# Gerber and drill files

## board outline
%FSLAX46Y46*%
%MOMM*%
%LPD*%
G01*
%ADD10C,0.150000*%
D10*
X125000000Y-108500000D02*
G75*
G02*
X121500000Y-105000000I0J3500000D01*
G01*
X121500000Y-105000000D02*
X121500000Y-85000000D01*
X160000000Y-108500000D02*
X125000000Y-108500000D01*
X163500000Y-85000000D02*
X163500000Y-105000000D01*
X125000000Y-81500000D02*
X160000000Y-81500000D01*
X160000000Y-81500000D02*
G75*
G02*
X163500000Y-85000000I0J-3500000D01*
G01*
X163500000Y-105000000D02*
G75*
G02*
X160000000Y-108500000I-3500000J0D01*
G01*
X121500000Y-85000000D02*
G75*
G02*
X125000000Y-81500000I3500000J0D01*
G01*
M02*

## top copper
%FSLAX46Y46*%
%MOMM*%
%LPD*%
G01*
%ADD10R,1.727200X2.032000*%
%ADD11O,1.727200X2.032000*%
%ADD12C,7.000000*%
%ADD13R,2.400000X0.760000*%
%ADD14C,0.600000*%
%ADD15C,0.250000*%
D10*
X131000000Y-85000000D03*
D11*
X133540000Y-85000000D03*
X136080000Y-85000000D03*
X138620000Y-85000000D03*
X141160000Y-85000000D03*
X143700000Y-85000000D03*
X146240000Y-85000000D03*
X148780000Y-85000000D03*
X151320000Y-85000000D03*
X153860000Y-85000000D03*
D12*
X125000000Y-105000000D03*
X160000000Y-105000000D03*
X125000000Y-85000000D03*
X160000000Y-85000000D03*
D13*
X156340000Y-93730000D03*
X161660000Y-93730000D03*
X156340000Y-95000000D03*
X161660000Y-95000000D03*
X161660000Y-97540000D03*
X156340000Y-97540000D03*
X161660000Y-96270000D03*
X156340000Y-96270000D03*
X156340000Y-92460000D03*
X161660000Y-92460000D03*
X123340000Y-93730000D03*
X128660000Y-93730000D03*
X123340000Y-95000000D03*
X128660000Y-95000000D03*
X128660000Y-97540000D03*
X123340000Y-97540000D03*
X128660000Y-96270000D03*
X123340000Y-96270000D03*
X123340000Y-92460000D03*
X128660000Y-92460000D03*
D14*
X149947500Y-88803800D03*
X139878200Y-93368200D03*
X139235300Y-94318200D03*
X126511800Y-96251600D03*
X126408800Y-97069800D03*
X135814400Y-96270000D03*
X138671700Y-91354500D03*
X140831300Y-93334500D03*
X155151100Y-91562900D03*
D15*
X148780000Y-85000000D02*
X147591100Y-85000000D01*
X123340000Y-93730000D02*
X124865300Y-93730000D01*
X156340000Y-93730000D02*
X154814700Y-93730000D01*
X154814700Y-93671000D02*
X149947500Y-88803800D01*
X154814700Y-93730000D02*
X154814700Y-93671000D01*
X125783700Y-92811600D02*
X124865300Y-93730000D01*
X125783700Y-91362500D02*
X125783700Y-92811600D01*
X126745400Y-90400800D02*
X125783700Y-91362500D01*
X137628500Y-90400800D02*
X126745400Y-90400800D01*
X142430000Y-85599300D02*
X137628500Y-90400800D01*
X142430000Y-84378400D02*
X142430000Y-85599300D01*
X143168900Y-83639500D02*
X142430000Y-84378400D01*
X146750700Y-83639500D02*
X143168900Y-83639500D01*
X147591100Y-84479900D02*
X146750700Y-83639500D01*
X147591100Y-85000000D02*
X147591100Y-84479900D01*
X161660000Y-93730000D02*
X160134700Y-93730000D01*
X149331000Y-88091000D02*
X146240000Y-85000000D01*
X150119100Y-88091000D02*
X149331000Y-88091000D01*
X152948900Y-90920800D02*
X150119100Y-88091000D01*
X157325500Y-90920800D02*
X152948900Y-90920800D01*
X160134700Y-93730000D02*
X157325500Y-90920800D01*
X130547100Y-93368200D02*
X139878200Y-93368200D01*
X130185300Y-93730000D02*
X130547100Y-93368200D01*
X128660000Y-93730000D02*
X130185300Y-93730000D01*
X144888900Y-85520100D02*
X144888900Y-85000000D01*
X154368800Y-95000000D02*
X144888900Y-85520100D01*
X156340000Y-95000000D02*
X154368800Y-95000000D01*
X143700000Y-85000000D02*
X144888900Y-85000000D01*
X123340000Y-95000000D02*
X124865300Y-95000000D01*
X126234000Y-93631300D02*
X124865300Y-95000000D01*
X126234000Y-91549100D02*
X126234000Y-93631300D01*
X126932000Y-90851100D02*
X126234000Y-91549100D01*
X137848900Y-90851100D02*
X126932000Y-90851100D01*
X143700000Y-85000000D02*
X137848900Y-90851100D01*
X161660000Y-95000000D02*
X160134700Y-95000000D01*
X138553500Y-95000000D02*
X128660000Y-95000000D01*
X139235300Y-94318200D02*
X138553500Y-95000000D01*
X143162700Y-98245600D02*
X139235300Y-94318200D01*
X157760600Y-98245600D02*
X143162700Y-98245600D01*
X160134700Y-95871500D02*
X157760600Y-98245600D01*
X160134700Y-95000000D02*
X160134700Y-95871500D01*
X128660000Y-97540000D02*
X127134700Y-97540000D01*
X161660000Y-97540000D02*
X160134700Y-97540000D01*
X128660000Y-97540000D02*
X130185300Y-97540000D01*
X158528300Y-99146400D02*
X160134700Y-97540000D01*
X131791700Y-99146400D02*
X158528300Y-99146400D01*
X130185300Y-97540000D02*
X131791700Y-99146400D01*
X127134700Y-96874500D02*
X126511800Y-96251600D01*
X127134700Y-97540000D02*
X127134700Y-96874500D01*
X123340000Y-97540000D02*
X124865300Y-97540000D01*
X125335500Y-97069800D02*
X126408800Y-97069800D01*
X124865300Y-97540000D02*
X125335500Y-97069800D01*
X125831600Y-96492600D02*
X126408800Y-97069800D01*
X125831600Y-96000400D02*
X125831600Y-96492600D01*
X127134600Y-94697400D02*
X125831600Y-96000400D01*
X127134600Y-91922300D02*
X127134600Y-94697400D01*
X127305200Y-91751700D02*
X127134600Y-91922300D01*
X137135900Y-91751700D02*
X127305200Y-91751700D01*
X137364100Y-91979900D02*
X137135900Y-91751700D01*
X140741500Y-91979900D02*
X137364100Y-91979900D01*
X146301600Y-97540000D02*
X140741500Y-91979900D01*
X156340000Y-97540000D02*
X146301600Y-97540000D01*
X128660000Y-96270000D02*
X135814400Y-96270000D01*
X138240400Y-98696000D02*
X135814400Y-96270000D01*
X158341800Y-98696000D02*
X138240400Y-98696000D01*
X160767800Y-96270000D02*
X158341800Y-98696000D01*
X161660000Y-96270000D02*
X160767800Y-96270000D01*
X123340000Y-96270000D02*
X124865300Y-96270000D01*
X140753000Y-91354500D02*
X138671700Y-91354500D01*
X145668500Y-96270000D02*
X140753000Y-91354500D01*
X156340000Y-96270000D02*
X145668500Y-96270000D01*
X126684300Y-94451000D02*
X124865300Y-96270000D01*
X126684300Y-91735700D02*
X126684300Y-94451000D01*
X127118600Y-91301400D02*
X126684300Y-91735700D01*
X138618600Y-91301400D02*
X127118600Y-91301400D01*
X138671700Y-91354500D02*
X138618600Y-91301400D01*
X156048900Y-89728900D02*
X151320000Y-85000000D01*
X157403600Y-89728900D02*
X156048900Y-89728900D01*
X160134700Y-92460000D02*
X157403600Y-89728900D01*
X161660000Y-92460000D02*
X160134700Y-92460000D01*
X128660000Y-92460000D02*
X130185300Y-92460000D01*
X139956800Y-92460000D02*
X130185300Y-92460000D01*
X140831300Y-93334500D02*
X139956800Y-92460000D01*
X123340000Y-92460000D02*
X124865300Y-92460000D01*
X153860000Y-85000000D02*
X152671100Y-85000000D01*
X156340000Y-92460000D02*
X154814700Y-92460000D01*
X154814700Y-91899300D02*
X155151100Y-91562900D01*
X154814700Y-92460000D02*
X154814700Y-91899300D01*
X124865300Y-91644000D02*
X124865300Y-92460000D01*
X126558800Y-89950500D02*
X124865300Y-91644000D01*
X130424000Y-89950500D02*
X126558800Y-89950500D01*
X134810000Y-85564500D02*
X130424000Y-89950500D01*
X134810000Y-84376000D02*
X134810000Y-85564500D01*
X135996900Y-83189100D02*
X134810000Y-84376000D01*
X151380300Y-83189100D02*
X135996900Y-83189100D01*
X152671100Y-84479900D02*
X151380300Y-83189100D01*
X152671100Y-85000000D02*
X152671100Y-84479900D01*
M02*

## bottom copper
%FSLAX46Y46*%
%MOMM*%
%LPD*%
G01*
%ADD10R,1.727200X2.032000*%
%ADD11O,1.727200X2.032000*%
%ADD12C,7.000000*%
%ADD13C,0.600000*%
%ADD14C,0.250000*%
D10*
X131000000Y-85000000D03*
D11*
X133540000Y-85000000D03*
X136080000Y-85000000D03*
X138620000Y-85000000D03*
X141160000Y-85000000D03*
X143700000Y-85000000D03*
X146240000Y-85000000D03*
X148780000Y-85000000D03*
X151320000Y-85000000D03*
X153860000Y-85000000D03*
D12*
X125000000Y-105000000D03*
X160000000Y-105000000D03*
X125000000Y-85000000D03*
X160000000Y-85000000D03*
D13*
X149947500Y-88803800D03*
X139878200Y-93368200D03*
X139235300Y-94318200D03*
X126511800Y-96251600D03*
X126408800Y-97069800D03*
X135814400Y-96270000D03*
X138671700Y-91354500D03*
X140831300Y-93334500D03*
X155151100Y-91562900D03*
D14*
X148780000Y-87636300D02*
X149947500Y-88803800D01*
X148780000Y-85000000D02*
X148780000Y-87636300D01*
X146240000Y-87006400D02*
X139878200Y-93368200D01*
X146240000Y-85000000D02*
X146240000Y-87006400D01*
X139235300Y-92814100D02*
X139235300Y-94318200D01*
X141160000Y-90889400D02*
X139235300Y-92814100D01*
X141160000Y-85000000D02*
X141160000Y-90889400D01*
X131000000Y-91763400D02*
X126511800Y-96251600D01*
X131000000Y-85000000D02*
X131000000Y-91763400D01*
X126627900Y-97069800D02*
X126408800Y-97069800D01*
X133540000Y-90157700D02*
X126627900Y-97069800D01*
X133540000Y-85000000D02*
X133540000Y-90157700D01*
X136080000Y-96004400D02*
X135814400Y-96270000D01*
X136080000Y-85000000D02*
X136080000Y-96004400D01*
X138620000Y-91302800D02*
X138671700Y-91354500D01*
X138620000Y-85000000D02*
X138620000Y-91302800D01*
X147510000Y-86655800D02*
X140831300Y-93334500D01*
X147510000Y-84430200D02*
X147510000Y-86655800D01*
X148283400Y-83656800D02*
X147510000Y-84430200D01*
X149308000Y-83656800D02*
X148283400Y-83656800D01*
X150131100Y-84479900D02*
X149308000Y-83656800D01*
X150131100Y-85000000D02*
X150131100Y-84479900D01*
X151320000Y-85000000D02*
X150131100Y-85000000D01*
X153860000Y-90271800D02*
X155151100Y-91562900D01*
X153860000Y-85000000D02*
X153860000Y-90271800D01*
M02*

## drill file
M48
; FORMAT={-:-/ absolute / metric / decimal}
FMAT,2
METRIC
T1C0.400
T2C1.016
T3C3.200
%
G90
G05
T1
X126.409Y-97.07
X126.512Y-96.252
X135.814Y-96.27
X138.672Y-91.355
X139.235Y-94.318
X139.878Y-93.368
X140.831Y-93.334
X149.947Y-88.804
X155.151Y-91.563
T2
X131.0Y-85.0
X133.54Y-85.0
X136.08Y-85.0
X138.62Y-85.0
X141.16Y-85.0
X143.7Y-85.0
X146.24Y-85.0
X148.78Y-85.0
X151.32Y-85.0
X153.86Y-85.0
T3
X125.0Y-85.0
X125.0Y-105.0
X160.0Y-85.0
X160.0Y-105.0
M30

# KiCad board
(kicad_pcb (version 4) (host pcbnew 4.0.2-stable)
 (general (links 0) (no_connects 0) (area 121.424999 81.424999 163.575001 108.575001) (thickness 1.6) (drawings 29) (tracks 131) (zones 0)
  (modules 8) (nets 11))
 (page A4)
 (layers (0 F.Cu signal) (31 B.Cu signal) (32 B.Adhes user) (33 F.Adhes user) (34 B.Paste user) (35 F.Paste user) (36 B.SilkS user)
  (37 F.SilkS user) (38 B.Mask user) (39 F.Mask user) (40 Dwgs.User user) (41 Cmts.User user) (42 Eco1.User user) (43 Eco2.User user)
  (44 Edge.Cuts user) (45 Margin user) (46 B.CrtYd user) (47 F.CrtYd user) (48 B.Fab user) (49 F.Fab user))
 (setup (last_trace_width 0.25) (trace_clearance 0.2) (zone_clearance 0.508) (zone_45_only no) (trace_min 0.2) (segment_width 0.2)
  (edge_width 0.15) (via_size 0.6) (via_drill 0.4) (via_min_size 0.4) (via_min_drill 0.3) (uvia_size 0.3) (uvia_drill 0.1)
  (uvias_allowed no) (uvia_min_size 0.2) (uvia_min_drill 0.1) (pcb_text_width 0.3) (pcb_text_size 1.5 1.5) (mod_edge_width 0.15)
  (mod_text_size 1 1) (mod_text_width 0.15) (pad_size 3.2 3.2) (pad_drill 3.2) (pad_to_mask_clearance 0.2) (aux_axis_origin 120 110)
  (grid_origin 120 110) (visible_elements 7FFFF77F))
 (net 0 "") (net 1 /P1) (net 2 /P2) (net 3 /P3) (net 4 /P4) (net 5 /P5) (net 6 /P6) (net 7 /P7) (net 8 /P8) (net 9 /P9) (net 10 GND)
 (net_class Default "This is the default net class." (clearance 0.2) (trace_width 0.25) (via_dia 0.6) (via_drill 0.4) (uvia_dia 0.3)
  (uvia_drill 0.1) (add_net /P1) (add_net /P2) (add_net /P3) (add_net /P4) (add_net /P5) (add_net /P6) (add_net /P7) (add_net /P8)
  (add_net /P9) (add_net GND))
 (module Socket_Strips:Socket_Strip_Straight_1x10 (layer F.Cu) (at 131 85)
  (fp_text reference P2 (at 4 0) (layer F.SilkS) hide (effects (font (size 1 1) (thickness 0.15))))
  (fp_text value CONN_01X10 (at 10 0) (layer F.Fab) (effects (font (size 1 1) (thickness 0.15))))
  (pad 1 thru_hole rect (at 0 0) (size 1.7272 2.032) (drill 1.016) (layers *.Cu *.Mask F.SilkS) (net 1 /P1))
  (pad 2 thru_hole oval (at 2.54 0) (size 1.7272 2.032) (drill 1.016) (layers *.Cu *.Mask F.SilkS) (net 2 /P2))
  (pad 3 thru_hole oval (at 5.08 0) (size 1.7272 2.032) (drill 1.016) (layers *.Cu *.Mask F.SilkS) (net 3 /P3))
  (pad 4 thru_hole oval (at 7.62 0) (size 1.7272 2.032) (drill 1.016) (layers *.Cu *.Mask F.SilkS) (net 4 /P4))
  (pad 5 thru_hole oval (at 10.16 0) (size 1.7272 2.032) (drill 1.016) (layers *.Cu *.Mask F.SilkS) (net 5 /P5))
  (pad 6 thru_hole oval (at 12.7 0) (size 1.7272 2.032) (drill 1.016) (layers *.Cu *.Mask F.SilkS) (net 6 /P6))
  (pad 7 thru_hole oval (at 15.24 0) (size 1.7272 2.032) (drill 1.016) (layers *.Cu *.Mask F.SilkS) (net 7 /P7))
  (pad 8 thru_hole oval (at 17.78 0) (size 1.7272 2.032) (drill 1.016) (layers *.Cu *.Mask F.SilkS) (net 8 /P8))
  (pad 9 thru_hole oval (at 20.32 0) (size 1.7272 2.032) (drill 1.016) (layers *.Cu *.Mask F.SilkS) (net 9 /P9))
  (pad 10 thru_hole oval (at 22.86 0) (size 1.7272 2.032) (drill 1.016) (layers *.Cu *.Mask F.SilkS) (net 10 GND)))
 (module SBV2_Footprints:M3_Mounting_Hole (layer F.Cu) (at 125 105)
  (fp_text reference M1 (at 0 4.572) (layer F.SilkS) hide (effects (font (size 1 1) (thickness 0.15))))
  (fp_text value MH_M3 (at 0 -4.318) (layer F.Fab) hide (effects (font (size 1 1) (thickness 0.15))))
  (pad "" np_thru_hole circle (at 0 0) (size 7 7) (drill 3.2) (layers *.Cu *.Mask)))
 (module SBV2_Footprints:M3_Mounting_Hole (layer F.Cu) (at 160 105)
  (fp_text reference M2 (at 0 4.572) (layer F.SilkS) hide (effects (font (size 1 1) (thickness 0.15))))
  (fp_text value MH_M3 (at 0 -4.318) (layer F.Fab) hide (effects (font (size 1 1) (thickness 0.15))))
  (pad "" np_thru_hole circle (at 0 0) (size 7 7) (drill 3.2) (layers *.Cu *.Mask)))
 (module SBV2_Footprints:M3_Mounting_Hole (layer F.Cu) (at 125 85)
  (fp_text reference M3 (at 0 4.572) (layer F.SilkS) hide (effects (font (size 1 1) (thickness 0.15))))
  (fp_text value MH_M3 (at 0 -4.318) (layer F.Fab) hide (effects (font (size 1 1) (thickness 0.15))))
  (pad "" np_thru_hole circle (at 0 0) (size 7 7) (drill 3.2) (layers *.Cu *.Mask)))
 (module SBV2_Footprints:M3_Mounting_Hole (layer F.Cu) (at 160 85)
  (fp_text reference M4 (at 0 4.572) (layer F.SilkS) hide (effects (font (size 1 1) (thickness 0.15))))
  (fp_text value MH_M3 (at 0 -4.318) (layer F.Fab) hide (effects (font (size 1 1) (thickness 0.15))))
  (pad "" np_thru_hole circle (at 0 0) (size 7 7) (drill 3.2) (layers *.Cu *.Mask)))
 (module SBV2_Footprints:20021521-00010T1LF (layer F.Cu) (at 159 95 90)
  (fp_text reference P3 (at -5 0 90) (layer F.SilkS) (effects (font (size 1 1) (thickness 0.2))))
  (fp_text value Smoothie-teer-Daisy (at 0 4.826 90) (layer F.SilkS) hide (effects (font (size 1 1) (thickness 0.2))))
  (pad 8 smd rect (at 1.27 -2.66 90) (size 0.76 2.4) (layers F.Cu F.Paste F.Mask) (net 8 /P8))
  (pad 7 smd rect (at 1.27 2.66 90) (size 0.76 2.4) (layers F.Cu F.Paste F.Mask) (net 7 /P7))
  (pad 6 smd rect (at 0 -2.66 90) (size 0.76 2.4) (layers F.Cu F.Paste F.Mask) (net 6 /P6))
  (pad 5 smd rect (at 0 2.66 270) (size 0.76 2.4) (layers F.Cu F.Paste F.Mask) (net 5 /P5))
  (pad 1 smd rect (at -2.54 2.66 90) (size 0.76 2.4) (layers F.Cu F.Paste F.Mask) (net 1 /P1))
  (pad 2 smd rect (at -2.54 -2.66 90) (size 0.76 2.4) (layers F.Cu F.Paste F.Mask) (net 2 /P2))
  (pad 3 smd rect (at -1.27 2.66 90) (size 0.76 2.4) (layers F.Cu F.Paste F.Mask) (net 3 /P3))
  (pad 4 smd rect (at -1.27 -2.66 90) (size 0.76 2.4) (layers F.Cu F.Paste F.Mask) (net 4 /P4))
  (pad 10 smd rect (at 2.54 -2.66 90) (size 0.76 2.4) (layers F.Cu F.Paste F.Mask) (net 10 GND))
  (pad 9 smd rect (at 2.54 2.66 90) (size 0.76 2.4) (layers F.Cu F.Paste F.Mask) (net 9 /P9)))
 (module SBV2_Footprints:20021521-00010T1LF (layer F.Cu) (at 126 95 90)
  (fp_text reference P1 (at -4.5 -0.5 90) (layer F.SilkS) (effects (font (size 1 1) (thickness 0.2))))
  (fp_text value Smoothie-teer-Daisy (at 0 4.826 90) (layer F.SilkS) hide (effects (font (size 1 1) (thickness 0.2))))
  (pad 8 smd rect (at 1.27 -2.66 90) (size 0.76 2.4) (layers F.Cu F.Paste F.Mask) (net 8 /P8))
  (pad 7 smd rect (at 1.27 2.66 90) (size 0.76 2.4) (layers F.Cu F.Paste F.Mask) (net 7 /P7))
  (pad 6 smd rect (at 0 -2.66 90) (size 0.76 2.4) (layers F.Cu F.Paste F.Mask) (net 6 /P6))
  (pad 5 smd rect (at 0 2.66 270) (size 0.76 2.4) (layers F.Cu F.Paste F.Mask) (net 5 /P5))
  (pad 1 smd rect (at -2.54 2.66 90) (size 0.76 2.4) (layers F.Cu F.Paste F.Mask) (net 1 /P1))
  (pad 2 smd rect (at -2.54 -2.66 90) (size 0.76 2.4) (layers F.Cu F.Paste F.Mask) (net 2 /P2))
  (pad 3 smd rect (at -1.27 2.66 90) (size 0.76 2.4) (layers F.Cu F.Paste F.Mask) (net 3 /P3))
  (pad 4 smd rect (at -1.27 -2.66 90) (size 0.76 2.4) (layers F.Cu F.Paste F.Mask) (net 4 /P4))
  (pad 10 smd rect (at 2.54 -2.66 90) (size 0.76 2.4) (layers F.Cu F.Paste F.Mask) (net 10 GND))
  (pad 9 smd rect (at 2.54 2.66 90) (size 0.76 2.4) (layers F.Cu F.Paste F.Mask) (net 9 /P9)))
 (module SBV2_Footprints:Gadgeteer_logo (layer F.Cu) (at 143 98.25)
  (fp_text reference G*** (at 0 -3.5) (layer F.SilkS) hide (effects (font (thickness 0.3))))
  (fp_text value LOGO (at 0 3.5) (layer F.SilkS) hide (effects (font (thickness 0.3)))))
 (gr_arc (start 125 105) (end 125 108.5) (angle 90) (layer Edge.Cuts) (width 0.15))
 (gr_line (start 121.5 105) (end 121.5 85) (angle 90) (layer Edge.Cuts) (width 0.15))
 (gr_line (start 160 108.5) (end 125 108.5) (angle 90) (layer Edge.Cuts) (width 0.15))
 (gr_line (start 163.5 85) (end 163.5 105) (angle 90) (layer Edge.Cuts) (width 0.15))
 (gr_line (start 125 81.5) (end 160 81.5) (angle 90) (layer Edge.Cuts) (width 0.15))
 (gr_arc (start 160 85) (end 160 81.5) (angle 90) (layer Edge.Cuts) (width 0.15))
 (gr_arc (start 160 105) (end 163.5 105) (angle 90) (layer Edge.Cuts) (width 0.15))
 (gr_arc (start 125 85) (end 121.5 85) (angle 90) (layer Edge.Cuts) (width 0.15))
 (via (at 149.9475 88.8038) (size 0.6) (layers F.Cu B.Cu) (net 8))
 (segment (start 148.78 85) (end 147.5911 85) (width 0.25) (layer F.Cu) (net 8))
 (segment (start 123.34 93.73) (end 124.8653 93.73) (width 0.25) (layer F.Cu) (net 8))
 (segment (start 156.34 93.73) (end 154.8147 93.73) (width 0.25) (layer F.Cu) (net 8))
 (segment (start 148.78 87.6363) (end 149.9475 88.8038) (width 0.25) (layer B.Cu) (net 8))
 (segment (start 148.78 85) (end 148.78 87.6363) (width 0.25) (layer B.Cu) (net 8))
 (segment (start 154.8147 93.671) (end 149.9475 88.8038) (width 0.25) (layer F.Cu) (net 8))
 (segment (start 154.8147 93.73) (end 154.8147 93.671) (width 0.25) (layer F.Cu) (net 8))
 (segment (start 125.7837 92.8116) (end 124.8653 93.73) (width 0.25) (layer F.Cu) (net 8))
 (segment (start 125.7837 91.3625) (end 125.7837 92.8116) (width 0.25) (layer F.Cu) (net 8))
 (segment (start 126.7454 90.4008) (end 125.7837 91.3625) (width 0.25) (layer F.Cu) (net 8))
 (segment (start 137.6285 90.4008) (end 126.7454 90.4008) (width 0.25) (layer F.Cu) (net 8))
 (segment (start 142.43 85.5993) (end 137.6285 90.4008) (width 0.25) (layer F.Cu) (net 8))
 (segment (start 142.43 84.3784) (end 142.43 85.5993) (width 0.25) (layer F.Cu) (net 8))
 (segment (start 143.1689 83.6395) (end 142.43 84.3784) (width 0.25) (layer F.Cu) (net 8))
 (segment (start 146.7507 83.6395) (end 143.1689 83.6395) (width 0.25) (layer F.Cu) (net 8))
 (segment (start 147.5911 84.4799) (end 146.7507 83.6395) (width 0.25) (layer F.Cu) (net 8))
 (segment (start 147.5911 85) (end 147.5911 84.4799) (width 0.25) (layer F.Cu) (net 8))
 (via (at 139.8782 93.3682) (size 0.6) (layers F.Cu B.Cu) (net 7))
 (segment (start 161.66 93.73) (end 160.1347 93.73) (width 0.25) (layer F.Cu) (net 7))
 (segment (start 149.331 88.091) (end 146.24 85) (width 0.25) (layer F.Cu) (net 7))
 (segment (start 150.1191 88.091) (end 149.331 88.091) (width 0.25) (layer F.Cu) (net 7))
 (segment (start 152.9489 90.9208) (end 150.1191 88.091) (width 0.25) (layer F.Cu) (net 7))
 (segment (start 157.3255 90.9208) (end 152.9489 90.9208) (width 0.25) (layer F.Cu) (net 7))
 (segment (start 160.1347 93.73) (end 157.3255 90.9208) (width 0.25) (layer F.Cu) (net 7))
 (segment (start 130.5471 93.3682) (end 139.8782 93.3682) (width 0.25) (layer F.Cu) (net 7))
 (segment (start 130.1853 93.73) (end 130.5471 93.3682) (width 0.25) (layer F.Cu) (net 7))
 (segment (start 128.66 93.73) (end 130.1853 93.73) (width 0.25) (layer F.Cu) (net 7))
 (segment (start 146.24 87.0064) (end 139.8782 93.3682) (width 0.25) (layer B.Cu) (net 7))
 (segment (start 146.24 85) (end 146.24 87.0064) (width 0.25) (layer B.Cu) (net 7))
 (segment (start 144.8889 85.5201) (end 144.8889 85) (width 0.25) (layer F.Cu) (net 6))
 (segment (start 154.3688 95) (end 144.8889 85.5201) (width 0.25) (layer F.Cu) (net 6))
 (segment (start 156.34 95) (end 154.3688 95) (width 0.25) (layer F.Cu) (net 6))
 (segment (start 143.7 85) (end 144.8889 85) (width 0.25) (layer F.Cu) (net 6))
 (segment (start 123.34 95) (end 124.8653 95) (width 0.25) (layer F.Cu) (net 6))
 (segment (start 126.234 93.6313) (end 124.8653 95) (width 0.25) (layer F.Cu) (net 6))
 (segment (start 126.234 91.5491) (end 126.234 93.6313) (width 0.25) (layer F.Cu) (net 6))
 (segment (start 126.932 90.8511) (end 126.234 91.5491) (width 0.25) (layer F.Cu) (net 6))
 (segment (start 137.8489 90.8511) (end 126.932 90.8511) (width 0.25) (layer F.Cu) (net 6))
 (segment (start 143.7 85) (end 137.8489 90.8511) (width 0.25) (layer F.Cu) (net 6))
 (via (at 139.2353 94.3182) (size 0.6) (layers F.Cu B.Cu) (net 5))
 (segment (start 161.66 95) (end 160.1347 95) (width 0.25) (layer F.Cu) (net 5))
 (segment (start 139.2353 92.8141) (end 139.2353 94.3182) (width 0.25) (layer B.Cu) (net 5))
 (segment (start 141.16 90.8894) (end 139.2353 92.8141) (width 0.25) (layer B.Cu) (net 5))
 (segment (start 141.16 85) (end 141.16 90.8894) (width 0.25) (layer B.Cu) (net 5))
 (segment (start 138.5535 95) (end 128.66 95) (width 0.25) (layer F.Cu) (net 5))
 (segment (start 139.2353 94.3182) (end 138.5535 95) (width 0.25) (layer F.Cu) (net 5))
 (segment (start 143.1627 98.2456) (end 139.2353 94.3182) (width 0.25) (layer F.Cu) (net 5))
 (segment (start 157.7606 98.2456) (end 143.1627 98.2456) (width 0.25) (layer F.Cu) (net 5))
 (segment (start 160.1347 95.8715) (end 157.7606 98.2456) (width 0.25) (layer F.Cu) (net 5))
 (segment (start 160.1347 95) (end 160.1347 95.8715) (width 0.25) (layer F.Cu) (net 5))
 (via (at 126.5118 96.2516) (size 0.6) (layers F.Cu B.Cu) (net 1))
 (segment (start 128.66 97.54) (end 127.1347 97.54) (width 0.25) (layer F.Cu) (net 1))
 (segment (start 161.66 97.54) (end 160.1347 97.54) (width 0.25) (layer F.Cu) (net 1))
 (segment (start 128.66 97.54) (end 130.1853 97.54) (width 0.25) (layer F.Cu) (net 1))
 (segment (start 158.5283 99.1464) (end 160.1347 97.54) (width 0.25) (layer F.Cu) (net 1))
 (segment (start 131.7917 99.1464) (end 158.5283 99.1464) (width 0.25) (layer F.Cu) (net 1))
 (segment (start 130.1853 97.54) (end 131.7917 99.1464) (width 0.25) (layer F.Cu) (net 1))
 (segment (start 131 91.7634) (end 126.5118 96.2516) (width 0.25) (layer B.Cu) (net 1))
 (segment (start 131 85) (end 131 91.7634) (width 0.25) (layer B.Cu) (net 1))
 (segment (start 127.1347 96.8745) (end 126.5118 96.2516) (width 0.25) (layer F.Cu) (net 1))
 (segment (start 127.1347 97.54) (end 127.1347 96.8745) (width 0.25) (layer F.Cu) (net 1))
 (via (at 126.4088 97.0698) (size 0.6) (layers F.Cu B.Cu) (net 2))
 (segment (start 123.34 97.54) (end 124.8653 97.54) (width 0.25) (layer F.Cu) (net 2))
 (segment (start 125.3355 97.0698) (end 126.4088 97.0698) (width 0.25) (layer F.Cu) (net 2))
 (segment (start 124.8653 97.54) (end 125.3355 97.0698) (width 0.25) (layer F.Cu) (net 2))
 (segment (start 126.6279 97.0698) (end 126.4088 97.0698) (width 0.25) (layer B.Cu) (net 2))
 (segment (start 133.54 90.1577) (end 126.6279 97.0698) (width 0.25) (layer B.Cu) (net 2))
 (segment (start 133.54 85) (end 133.54 90.1577) (width 0.25) (layer B.Cu) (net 2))
 (segment (start 125.8316 96.4926) (end 126.4088 97.0698) (width 0.25) (layer F.Cu) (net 2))
 (segment (start 125.8316 96.0004) (end 125.8316 96.4926) (width 0.25) (layer F.Cu) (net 2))
 (segment (start 127.1346 94.6974) (end 125.8316 96.0004) (width 0.25) (layer F.Cu) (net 2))
 (segment (start 127.1346 91.9223) (end 127.1346 94.6974) (width 0.25) (layer F.Cu) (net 2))
 (segment (start 127.3052 91.7517) (end 127.1346 91.9223) (width 0.25) (layer F.Cu) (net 2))
 (segment (start 137.1359 91.7517) (end 127.3052 91.7517) (width 0.25) (layer F.Cu) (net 2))
 (segment (start 137.3641 91.9799) (end 137.1359 91.7517) (width 0.25) (layer F.Cu) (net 2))
 (segment (start 140.7415 91.9799) (end 137.3641 91.9799) (width 0.25) (layer F.Cu) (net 2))
 (segment (start 146.3016 97.54) (end 140.7415 91.9799) (width 0.25) (layer F.Cu) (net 2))
 (segment (start 156.34 97.54) (end 146.3016 97.54) (width 0.25) (layer F.Cu) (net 2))
 (via (at 135.8144 96.27) (size 0.6) (layers F.Cu B.Cu) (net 3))
 (segment (start 136.08 96.0044) (end 135.8144 96.27) (width 0.25) (layer B.Cu) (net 3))
 (segment (start 136.08 85) (end 136.08 96.0044) (width 0.25) (layer B.Cu) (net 3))
 (segment (start 128.66 96.27) (end 135.8144 96.27) (width 0.25) (layer F.Cu) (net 3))
 (segment (start 138.2404 98.696) (end 135.8144 96.27) (width 0.25) (layer F.Cu) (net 3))
 (segment (start 158.3418 98.696) (end 138.2404 98.696) (width 0.25) (layer F.Cu) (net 3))
 (segment (start 160.7678 96.27) (end 158.3418 98.696) (width 0.25) (layer F.Cu) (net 3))
 (segment (start 161.66 96.27) (end 160.7678 96.27) (width 0.25) (layer F.Cu) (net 3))
 (via (at 138.6717 91.3545) (size 0.6) (layers F.Cu B.Cu) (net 4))
 (segment (start 123.34 96.27) (end 124.8653 96.27) (width 0.25) (layer F.Cu) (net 4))
 (segment (start 138.62 91.3028) (end 138.6717 91.3545) (width 0.25) (layer B.Cu) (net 4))
 (segment (start 138.62 85) (end 138.62 91.3028) (width 0.25) (layer B.Cu) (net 4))
 (segment (start 140.753 91.3545) (end 138.6717 91.3545) (width 0.25) (layer F.Cu) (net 4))
 (segment (start 145.6685 96.27) (end 140.753 91.3545) (width 0.25) (layer F.Cu) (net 4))
 (segment (start 156.34 96.27) (end 145.6685 96.27) (width 0.25) (layer F.Cu) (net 4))
 (segment (start 126.6843 94.451) (end 124.8653 96.27) (width 0.25) (layer F.Cu) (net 4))
 (segment (start 126.6843 91.7357) (end 126.6843 94.451) (width 0.25) (layer F.Cu) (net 4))
 (segment (start 127.1186 91.3014) (end 126.6843 91.7357) (width 0.25) (layer F.Cu) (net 4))
 (segment (start 138.6186 91.3014) (end 127.1186 91.3014) (width 0.25) (layer F.Cu) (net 4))
 (segment (start 138.6717 91.3545) (end 138.6186 91.3014) (width 0.25) (layer F.Cu) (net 4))
 (via (at 140.8313 93.3345) (size 0.6) (layers F.Cu B.Cu) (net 9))
 (segment (start 156.0489 89.7289) (end 151.32 85) (width 0.25) (layer F.Cu) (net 9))
 (segment (start 157.4036 89.7289) (end 156.0489 89.7289) (width 0.25) (layer F.Cu) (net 9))
 (segment (start 160.1347 92.46) (end 157.4036 89.7289) (width 0.25) (layer F.Cu) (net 9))
 (segment (start 161.66 92.46) (end 160.1347 92.46) (width 0.25) (layer F.Cu) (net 9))
 (segment (start 128.66 92.46) (end 130.1853 92.46) (width 0.25) (layer F.Cu) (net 9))
 (segment (start 147.51 86.6558) (end 140.8313 93.3345) (width 0.25) (layer B.Cu) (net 9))
 (segment (start 147.51 84.4302) (end 147.51 86.6558) (width 0.25) (layer B.Cu) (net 9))
 (segment (start 148.2834 83.6568) (end 147.51 84.4302) (width 0.25) (layer B.Cu) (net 9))
 (segment (start 149.308 83.6568) (end 148.2834 83.6568) (width 0.25) (layer B.Cu) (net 9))
 (segment (start 150.1311 84.4799) (end 149.308 83.6568) (width 0.25) (layer B.Cu) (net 9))
 (segment (start 150.1311 85) (end 150.1311 84.4799) (width 0.25) (layer B.Cu) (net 9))
 (segment (start 139.9568 92.46) (end 130.1853 92.46) (width 0.25) (layer F.Cu) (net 9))
 (segment (start 140.8313 93.3345) (end 139.9568 92.46) (width 0.25) (layer F.Cu) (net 9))
 (segment (start 151.32 85) (end 150.1311 85) (width 0.25) (layer B.Cu) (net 9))
 (via (at 155.1511 91.5629) (size 0.6) (layers F.Cu B.Cu) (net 10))
 (segment (start 123.34 92.46) (end 124.8653 92.46) (width 0.25) (layer F.Cu) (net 10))
 (segment (start 153.86 85) (end 152.6711 85) (width 0.25) (layer F.Cu) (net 10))
 (segment (start 156.34 92.46) (end 154.8147 92.46) (width 0.25) (layer F.Cu) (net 10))
 (segment (start 153.86 90.2718) (end 155.1511 91.5629) (width 0.25) (layer B.Cu) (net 10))
 (segment (start 153.86 85) (end 153.86 90.2718) (width 0.25) (layer B.Cu) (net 10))
 (segment (start 154.8147 91.8993) (end 155.1511 91.5629) (width 0.25) (layer F.Cu) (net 10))
 (segment (start 154.8147 92.46) (end 154.8147 91.8993) (width 0.25) (layer F.Cu) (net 10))
 (segment (start 124.8653 91.644) (end 124.8653 92.46) (width 0.25) (layer F.Cu) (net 10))
 (segment (start 126.5588 89.9505) (end 124.8653 91.644) (width 0.25) (layer F.Cu) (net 10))
 (segment (start 130.424 89.9505) (end 126.5588 89.9505) (width 0.25) (layer F.Cu) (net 10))
 (segment (start 134.81 85.5645) (end 130.424 89.9505) (width 0.25) (layer F.Cu) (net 10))
 (segment (start 134.81 84.376) (end 134.81 85.5645) (width 0.25) (layer F.Cu) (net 10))
 (segment (start 135.9969 83.1891) (end 134.81 84.376) (width 0.25) (layer F.Cu) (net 10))
 (segment (start 151.3803 83.1891) (end 135.9969 83.1891) (width 0.25) (layer F.Cu) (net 10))
 (segment (start 152.6711 84.4799) (end 151.3803 83.1891) (width 0.25) (layer F.Cu) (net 10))
 (segment (start 152.6711 85) (end 152.6711 84.4799) (width 0.25) (layer F.Cu) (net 10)))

